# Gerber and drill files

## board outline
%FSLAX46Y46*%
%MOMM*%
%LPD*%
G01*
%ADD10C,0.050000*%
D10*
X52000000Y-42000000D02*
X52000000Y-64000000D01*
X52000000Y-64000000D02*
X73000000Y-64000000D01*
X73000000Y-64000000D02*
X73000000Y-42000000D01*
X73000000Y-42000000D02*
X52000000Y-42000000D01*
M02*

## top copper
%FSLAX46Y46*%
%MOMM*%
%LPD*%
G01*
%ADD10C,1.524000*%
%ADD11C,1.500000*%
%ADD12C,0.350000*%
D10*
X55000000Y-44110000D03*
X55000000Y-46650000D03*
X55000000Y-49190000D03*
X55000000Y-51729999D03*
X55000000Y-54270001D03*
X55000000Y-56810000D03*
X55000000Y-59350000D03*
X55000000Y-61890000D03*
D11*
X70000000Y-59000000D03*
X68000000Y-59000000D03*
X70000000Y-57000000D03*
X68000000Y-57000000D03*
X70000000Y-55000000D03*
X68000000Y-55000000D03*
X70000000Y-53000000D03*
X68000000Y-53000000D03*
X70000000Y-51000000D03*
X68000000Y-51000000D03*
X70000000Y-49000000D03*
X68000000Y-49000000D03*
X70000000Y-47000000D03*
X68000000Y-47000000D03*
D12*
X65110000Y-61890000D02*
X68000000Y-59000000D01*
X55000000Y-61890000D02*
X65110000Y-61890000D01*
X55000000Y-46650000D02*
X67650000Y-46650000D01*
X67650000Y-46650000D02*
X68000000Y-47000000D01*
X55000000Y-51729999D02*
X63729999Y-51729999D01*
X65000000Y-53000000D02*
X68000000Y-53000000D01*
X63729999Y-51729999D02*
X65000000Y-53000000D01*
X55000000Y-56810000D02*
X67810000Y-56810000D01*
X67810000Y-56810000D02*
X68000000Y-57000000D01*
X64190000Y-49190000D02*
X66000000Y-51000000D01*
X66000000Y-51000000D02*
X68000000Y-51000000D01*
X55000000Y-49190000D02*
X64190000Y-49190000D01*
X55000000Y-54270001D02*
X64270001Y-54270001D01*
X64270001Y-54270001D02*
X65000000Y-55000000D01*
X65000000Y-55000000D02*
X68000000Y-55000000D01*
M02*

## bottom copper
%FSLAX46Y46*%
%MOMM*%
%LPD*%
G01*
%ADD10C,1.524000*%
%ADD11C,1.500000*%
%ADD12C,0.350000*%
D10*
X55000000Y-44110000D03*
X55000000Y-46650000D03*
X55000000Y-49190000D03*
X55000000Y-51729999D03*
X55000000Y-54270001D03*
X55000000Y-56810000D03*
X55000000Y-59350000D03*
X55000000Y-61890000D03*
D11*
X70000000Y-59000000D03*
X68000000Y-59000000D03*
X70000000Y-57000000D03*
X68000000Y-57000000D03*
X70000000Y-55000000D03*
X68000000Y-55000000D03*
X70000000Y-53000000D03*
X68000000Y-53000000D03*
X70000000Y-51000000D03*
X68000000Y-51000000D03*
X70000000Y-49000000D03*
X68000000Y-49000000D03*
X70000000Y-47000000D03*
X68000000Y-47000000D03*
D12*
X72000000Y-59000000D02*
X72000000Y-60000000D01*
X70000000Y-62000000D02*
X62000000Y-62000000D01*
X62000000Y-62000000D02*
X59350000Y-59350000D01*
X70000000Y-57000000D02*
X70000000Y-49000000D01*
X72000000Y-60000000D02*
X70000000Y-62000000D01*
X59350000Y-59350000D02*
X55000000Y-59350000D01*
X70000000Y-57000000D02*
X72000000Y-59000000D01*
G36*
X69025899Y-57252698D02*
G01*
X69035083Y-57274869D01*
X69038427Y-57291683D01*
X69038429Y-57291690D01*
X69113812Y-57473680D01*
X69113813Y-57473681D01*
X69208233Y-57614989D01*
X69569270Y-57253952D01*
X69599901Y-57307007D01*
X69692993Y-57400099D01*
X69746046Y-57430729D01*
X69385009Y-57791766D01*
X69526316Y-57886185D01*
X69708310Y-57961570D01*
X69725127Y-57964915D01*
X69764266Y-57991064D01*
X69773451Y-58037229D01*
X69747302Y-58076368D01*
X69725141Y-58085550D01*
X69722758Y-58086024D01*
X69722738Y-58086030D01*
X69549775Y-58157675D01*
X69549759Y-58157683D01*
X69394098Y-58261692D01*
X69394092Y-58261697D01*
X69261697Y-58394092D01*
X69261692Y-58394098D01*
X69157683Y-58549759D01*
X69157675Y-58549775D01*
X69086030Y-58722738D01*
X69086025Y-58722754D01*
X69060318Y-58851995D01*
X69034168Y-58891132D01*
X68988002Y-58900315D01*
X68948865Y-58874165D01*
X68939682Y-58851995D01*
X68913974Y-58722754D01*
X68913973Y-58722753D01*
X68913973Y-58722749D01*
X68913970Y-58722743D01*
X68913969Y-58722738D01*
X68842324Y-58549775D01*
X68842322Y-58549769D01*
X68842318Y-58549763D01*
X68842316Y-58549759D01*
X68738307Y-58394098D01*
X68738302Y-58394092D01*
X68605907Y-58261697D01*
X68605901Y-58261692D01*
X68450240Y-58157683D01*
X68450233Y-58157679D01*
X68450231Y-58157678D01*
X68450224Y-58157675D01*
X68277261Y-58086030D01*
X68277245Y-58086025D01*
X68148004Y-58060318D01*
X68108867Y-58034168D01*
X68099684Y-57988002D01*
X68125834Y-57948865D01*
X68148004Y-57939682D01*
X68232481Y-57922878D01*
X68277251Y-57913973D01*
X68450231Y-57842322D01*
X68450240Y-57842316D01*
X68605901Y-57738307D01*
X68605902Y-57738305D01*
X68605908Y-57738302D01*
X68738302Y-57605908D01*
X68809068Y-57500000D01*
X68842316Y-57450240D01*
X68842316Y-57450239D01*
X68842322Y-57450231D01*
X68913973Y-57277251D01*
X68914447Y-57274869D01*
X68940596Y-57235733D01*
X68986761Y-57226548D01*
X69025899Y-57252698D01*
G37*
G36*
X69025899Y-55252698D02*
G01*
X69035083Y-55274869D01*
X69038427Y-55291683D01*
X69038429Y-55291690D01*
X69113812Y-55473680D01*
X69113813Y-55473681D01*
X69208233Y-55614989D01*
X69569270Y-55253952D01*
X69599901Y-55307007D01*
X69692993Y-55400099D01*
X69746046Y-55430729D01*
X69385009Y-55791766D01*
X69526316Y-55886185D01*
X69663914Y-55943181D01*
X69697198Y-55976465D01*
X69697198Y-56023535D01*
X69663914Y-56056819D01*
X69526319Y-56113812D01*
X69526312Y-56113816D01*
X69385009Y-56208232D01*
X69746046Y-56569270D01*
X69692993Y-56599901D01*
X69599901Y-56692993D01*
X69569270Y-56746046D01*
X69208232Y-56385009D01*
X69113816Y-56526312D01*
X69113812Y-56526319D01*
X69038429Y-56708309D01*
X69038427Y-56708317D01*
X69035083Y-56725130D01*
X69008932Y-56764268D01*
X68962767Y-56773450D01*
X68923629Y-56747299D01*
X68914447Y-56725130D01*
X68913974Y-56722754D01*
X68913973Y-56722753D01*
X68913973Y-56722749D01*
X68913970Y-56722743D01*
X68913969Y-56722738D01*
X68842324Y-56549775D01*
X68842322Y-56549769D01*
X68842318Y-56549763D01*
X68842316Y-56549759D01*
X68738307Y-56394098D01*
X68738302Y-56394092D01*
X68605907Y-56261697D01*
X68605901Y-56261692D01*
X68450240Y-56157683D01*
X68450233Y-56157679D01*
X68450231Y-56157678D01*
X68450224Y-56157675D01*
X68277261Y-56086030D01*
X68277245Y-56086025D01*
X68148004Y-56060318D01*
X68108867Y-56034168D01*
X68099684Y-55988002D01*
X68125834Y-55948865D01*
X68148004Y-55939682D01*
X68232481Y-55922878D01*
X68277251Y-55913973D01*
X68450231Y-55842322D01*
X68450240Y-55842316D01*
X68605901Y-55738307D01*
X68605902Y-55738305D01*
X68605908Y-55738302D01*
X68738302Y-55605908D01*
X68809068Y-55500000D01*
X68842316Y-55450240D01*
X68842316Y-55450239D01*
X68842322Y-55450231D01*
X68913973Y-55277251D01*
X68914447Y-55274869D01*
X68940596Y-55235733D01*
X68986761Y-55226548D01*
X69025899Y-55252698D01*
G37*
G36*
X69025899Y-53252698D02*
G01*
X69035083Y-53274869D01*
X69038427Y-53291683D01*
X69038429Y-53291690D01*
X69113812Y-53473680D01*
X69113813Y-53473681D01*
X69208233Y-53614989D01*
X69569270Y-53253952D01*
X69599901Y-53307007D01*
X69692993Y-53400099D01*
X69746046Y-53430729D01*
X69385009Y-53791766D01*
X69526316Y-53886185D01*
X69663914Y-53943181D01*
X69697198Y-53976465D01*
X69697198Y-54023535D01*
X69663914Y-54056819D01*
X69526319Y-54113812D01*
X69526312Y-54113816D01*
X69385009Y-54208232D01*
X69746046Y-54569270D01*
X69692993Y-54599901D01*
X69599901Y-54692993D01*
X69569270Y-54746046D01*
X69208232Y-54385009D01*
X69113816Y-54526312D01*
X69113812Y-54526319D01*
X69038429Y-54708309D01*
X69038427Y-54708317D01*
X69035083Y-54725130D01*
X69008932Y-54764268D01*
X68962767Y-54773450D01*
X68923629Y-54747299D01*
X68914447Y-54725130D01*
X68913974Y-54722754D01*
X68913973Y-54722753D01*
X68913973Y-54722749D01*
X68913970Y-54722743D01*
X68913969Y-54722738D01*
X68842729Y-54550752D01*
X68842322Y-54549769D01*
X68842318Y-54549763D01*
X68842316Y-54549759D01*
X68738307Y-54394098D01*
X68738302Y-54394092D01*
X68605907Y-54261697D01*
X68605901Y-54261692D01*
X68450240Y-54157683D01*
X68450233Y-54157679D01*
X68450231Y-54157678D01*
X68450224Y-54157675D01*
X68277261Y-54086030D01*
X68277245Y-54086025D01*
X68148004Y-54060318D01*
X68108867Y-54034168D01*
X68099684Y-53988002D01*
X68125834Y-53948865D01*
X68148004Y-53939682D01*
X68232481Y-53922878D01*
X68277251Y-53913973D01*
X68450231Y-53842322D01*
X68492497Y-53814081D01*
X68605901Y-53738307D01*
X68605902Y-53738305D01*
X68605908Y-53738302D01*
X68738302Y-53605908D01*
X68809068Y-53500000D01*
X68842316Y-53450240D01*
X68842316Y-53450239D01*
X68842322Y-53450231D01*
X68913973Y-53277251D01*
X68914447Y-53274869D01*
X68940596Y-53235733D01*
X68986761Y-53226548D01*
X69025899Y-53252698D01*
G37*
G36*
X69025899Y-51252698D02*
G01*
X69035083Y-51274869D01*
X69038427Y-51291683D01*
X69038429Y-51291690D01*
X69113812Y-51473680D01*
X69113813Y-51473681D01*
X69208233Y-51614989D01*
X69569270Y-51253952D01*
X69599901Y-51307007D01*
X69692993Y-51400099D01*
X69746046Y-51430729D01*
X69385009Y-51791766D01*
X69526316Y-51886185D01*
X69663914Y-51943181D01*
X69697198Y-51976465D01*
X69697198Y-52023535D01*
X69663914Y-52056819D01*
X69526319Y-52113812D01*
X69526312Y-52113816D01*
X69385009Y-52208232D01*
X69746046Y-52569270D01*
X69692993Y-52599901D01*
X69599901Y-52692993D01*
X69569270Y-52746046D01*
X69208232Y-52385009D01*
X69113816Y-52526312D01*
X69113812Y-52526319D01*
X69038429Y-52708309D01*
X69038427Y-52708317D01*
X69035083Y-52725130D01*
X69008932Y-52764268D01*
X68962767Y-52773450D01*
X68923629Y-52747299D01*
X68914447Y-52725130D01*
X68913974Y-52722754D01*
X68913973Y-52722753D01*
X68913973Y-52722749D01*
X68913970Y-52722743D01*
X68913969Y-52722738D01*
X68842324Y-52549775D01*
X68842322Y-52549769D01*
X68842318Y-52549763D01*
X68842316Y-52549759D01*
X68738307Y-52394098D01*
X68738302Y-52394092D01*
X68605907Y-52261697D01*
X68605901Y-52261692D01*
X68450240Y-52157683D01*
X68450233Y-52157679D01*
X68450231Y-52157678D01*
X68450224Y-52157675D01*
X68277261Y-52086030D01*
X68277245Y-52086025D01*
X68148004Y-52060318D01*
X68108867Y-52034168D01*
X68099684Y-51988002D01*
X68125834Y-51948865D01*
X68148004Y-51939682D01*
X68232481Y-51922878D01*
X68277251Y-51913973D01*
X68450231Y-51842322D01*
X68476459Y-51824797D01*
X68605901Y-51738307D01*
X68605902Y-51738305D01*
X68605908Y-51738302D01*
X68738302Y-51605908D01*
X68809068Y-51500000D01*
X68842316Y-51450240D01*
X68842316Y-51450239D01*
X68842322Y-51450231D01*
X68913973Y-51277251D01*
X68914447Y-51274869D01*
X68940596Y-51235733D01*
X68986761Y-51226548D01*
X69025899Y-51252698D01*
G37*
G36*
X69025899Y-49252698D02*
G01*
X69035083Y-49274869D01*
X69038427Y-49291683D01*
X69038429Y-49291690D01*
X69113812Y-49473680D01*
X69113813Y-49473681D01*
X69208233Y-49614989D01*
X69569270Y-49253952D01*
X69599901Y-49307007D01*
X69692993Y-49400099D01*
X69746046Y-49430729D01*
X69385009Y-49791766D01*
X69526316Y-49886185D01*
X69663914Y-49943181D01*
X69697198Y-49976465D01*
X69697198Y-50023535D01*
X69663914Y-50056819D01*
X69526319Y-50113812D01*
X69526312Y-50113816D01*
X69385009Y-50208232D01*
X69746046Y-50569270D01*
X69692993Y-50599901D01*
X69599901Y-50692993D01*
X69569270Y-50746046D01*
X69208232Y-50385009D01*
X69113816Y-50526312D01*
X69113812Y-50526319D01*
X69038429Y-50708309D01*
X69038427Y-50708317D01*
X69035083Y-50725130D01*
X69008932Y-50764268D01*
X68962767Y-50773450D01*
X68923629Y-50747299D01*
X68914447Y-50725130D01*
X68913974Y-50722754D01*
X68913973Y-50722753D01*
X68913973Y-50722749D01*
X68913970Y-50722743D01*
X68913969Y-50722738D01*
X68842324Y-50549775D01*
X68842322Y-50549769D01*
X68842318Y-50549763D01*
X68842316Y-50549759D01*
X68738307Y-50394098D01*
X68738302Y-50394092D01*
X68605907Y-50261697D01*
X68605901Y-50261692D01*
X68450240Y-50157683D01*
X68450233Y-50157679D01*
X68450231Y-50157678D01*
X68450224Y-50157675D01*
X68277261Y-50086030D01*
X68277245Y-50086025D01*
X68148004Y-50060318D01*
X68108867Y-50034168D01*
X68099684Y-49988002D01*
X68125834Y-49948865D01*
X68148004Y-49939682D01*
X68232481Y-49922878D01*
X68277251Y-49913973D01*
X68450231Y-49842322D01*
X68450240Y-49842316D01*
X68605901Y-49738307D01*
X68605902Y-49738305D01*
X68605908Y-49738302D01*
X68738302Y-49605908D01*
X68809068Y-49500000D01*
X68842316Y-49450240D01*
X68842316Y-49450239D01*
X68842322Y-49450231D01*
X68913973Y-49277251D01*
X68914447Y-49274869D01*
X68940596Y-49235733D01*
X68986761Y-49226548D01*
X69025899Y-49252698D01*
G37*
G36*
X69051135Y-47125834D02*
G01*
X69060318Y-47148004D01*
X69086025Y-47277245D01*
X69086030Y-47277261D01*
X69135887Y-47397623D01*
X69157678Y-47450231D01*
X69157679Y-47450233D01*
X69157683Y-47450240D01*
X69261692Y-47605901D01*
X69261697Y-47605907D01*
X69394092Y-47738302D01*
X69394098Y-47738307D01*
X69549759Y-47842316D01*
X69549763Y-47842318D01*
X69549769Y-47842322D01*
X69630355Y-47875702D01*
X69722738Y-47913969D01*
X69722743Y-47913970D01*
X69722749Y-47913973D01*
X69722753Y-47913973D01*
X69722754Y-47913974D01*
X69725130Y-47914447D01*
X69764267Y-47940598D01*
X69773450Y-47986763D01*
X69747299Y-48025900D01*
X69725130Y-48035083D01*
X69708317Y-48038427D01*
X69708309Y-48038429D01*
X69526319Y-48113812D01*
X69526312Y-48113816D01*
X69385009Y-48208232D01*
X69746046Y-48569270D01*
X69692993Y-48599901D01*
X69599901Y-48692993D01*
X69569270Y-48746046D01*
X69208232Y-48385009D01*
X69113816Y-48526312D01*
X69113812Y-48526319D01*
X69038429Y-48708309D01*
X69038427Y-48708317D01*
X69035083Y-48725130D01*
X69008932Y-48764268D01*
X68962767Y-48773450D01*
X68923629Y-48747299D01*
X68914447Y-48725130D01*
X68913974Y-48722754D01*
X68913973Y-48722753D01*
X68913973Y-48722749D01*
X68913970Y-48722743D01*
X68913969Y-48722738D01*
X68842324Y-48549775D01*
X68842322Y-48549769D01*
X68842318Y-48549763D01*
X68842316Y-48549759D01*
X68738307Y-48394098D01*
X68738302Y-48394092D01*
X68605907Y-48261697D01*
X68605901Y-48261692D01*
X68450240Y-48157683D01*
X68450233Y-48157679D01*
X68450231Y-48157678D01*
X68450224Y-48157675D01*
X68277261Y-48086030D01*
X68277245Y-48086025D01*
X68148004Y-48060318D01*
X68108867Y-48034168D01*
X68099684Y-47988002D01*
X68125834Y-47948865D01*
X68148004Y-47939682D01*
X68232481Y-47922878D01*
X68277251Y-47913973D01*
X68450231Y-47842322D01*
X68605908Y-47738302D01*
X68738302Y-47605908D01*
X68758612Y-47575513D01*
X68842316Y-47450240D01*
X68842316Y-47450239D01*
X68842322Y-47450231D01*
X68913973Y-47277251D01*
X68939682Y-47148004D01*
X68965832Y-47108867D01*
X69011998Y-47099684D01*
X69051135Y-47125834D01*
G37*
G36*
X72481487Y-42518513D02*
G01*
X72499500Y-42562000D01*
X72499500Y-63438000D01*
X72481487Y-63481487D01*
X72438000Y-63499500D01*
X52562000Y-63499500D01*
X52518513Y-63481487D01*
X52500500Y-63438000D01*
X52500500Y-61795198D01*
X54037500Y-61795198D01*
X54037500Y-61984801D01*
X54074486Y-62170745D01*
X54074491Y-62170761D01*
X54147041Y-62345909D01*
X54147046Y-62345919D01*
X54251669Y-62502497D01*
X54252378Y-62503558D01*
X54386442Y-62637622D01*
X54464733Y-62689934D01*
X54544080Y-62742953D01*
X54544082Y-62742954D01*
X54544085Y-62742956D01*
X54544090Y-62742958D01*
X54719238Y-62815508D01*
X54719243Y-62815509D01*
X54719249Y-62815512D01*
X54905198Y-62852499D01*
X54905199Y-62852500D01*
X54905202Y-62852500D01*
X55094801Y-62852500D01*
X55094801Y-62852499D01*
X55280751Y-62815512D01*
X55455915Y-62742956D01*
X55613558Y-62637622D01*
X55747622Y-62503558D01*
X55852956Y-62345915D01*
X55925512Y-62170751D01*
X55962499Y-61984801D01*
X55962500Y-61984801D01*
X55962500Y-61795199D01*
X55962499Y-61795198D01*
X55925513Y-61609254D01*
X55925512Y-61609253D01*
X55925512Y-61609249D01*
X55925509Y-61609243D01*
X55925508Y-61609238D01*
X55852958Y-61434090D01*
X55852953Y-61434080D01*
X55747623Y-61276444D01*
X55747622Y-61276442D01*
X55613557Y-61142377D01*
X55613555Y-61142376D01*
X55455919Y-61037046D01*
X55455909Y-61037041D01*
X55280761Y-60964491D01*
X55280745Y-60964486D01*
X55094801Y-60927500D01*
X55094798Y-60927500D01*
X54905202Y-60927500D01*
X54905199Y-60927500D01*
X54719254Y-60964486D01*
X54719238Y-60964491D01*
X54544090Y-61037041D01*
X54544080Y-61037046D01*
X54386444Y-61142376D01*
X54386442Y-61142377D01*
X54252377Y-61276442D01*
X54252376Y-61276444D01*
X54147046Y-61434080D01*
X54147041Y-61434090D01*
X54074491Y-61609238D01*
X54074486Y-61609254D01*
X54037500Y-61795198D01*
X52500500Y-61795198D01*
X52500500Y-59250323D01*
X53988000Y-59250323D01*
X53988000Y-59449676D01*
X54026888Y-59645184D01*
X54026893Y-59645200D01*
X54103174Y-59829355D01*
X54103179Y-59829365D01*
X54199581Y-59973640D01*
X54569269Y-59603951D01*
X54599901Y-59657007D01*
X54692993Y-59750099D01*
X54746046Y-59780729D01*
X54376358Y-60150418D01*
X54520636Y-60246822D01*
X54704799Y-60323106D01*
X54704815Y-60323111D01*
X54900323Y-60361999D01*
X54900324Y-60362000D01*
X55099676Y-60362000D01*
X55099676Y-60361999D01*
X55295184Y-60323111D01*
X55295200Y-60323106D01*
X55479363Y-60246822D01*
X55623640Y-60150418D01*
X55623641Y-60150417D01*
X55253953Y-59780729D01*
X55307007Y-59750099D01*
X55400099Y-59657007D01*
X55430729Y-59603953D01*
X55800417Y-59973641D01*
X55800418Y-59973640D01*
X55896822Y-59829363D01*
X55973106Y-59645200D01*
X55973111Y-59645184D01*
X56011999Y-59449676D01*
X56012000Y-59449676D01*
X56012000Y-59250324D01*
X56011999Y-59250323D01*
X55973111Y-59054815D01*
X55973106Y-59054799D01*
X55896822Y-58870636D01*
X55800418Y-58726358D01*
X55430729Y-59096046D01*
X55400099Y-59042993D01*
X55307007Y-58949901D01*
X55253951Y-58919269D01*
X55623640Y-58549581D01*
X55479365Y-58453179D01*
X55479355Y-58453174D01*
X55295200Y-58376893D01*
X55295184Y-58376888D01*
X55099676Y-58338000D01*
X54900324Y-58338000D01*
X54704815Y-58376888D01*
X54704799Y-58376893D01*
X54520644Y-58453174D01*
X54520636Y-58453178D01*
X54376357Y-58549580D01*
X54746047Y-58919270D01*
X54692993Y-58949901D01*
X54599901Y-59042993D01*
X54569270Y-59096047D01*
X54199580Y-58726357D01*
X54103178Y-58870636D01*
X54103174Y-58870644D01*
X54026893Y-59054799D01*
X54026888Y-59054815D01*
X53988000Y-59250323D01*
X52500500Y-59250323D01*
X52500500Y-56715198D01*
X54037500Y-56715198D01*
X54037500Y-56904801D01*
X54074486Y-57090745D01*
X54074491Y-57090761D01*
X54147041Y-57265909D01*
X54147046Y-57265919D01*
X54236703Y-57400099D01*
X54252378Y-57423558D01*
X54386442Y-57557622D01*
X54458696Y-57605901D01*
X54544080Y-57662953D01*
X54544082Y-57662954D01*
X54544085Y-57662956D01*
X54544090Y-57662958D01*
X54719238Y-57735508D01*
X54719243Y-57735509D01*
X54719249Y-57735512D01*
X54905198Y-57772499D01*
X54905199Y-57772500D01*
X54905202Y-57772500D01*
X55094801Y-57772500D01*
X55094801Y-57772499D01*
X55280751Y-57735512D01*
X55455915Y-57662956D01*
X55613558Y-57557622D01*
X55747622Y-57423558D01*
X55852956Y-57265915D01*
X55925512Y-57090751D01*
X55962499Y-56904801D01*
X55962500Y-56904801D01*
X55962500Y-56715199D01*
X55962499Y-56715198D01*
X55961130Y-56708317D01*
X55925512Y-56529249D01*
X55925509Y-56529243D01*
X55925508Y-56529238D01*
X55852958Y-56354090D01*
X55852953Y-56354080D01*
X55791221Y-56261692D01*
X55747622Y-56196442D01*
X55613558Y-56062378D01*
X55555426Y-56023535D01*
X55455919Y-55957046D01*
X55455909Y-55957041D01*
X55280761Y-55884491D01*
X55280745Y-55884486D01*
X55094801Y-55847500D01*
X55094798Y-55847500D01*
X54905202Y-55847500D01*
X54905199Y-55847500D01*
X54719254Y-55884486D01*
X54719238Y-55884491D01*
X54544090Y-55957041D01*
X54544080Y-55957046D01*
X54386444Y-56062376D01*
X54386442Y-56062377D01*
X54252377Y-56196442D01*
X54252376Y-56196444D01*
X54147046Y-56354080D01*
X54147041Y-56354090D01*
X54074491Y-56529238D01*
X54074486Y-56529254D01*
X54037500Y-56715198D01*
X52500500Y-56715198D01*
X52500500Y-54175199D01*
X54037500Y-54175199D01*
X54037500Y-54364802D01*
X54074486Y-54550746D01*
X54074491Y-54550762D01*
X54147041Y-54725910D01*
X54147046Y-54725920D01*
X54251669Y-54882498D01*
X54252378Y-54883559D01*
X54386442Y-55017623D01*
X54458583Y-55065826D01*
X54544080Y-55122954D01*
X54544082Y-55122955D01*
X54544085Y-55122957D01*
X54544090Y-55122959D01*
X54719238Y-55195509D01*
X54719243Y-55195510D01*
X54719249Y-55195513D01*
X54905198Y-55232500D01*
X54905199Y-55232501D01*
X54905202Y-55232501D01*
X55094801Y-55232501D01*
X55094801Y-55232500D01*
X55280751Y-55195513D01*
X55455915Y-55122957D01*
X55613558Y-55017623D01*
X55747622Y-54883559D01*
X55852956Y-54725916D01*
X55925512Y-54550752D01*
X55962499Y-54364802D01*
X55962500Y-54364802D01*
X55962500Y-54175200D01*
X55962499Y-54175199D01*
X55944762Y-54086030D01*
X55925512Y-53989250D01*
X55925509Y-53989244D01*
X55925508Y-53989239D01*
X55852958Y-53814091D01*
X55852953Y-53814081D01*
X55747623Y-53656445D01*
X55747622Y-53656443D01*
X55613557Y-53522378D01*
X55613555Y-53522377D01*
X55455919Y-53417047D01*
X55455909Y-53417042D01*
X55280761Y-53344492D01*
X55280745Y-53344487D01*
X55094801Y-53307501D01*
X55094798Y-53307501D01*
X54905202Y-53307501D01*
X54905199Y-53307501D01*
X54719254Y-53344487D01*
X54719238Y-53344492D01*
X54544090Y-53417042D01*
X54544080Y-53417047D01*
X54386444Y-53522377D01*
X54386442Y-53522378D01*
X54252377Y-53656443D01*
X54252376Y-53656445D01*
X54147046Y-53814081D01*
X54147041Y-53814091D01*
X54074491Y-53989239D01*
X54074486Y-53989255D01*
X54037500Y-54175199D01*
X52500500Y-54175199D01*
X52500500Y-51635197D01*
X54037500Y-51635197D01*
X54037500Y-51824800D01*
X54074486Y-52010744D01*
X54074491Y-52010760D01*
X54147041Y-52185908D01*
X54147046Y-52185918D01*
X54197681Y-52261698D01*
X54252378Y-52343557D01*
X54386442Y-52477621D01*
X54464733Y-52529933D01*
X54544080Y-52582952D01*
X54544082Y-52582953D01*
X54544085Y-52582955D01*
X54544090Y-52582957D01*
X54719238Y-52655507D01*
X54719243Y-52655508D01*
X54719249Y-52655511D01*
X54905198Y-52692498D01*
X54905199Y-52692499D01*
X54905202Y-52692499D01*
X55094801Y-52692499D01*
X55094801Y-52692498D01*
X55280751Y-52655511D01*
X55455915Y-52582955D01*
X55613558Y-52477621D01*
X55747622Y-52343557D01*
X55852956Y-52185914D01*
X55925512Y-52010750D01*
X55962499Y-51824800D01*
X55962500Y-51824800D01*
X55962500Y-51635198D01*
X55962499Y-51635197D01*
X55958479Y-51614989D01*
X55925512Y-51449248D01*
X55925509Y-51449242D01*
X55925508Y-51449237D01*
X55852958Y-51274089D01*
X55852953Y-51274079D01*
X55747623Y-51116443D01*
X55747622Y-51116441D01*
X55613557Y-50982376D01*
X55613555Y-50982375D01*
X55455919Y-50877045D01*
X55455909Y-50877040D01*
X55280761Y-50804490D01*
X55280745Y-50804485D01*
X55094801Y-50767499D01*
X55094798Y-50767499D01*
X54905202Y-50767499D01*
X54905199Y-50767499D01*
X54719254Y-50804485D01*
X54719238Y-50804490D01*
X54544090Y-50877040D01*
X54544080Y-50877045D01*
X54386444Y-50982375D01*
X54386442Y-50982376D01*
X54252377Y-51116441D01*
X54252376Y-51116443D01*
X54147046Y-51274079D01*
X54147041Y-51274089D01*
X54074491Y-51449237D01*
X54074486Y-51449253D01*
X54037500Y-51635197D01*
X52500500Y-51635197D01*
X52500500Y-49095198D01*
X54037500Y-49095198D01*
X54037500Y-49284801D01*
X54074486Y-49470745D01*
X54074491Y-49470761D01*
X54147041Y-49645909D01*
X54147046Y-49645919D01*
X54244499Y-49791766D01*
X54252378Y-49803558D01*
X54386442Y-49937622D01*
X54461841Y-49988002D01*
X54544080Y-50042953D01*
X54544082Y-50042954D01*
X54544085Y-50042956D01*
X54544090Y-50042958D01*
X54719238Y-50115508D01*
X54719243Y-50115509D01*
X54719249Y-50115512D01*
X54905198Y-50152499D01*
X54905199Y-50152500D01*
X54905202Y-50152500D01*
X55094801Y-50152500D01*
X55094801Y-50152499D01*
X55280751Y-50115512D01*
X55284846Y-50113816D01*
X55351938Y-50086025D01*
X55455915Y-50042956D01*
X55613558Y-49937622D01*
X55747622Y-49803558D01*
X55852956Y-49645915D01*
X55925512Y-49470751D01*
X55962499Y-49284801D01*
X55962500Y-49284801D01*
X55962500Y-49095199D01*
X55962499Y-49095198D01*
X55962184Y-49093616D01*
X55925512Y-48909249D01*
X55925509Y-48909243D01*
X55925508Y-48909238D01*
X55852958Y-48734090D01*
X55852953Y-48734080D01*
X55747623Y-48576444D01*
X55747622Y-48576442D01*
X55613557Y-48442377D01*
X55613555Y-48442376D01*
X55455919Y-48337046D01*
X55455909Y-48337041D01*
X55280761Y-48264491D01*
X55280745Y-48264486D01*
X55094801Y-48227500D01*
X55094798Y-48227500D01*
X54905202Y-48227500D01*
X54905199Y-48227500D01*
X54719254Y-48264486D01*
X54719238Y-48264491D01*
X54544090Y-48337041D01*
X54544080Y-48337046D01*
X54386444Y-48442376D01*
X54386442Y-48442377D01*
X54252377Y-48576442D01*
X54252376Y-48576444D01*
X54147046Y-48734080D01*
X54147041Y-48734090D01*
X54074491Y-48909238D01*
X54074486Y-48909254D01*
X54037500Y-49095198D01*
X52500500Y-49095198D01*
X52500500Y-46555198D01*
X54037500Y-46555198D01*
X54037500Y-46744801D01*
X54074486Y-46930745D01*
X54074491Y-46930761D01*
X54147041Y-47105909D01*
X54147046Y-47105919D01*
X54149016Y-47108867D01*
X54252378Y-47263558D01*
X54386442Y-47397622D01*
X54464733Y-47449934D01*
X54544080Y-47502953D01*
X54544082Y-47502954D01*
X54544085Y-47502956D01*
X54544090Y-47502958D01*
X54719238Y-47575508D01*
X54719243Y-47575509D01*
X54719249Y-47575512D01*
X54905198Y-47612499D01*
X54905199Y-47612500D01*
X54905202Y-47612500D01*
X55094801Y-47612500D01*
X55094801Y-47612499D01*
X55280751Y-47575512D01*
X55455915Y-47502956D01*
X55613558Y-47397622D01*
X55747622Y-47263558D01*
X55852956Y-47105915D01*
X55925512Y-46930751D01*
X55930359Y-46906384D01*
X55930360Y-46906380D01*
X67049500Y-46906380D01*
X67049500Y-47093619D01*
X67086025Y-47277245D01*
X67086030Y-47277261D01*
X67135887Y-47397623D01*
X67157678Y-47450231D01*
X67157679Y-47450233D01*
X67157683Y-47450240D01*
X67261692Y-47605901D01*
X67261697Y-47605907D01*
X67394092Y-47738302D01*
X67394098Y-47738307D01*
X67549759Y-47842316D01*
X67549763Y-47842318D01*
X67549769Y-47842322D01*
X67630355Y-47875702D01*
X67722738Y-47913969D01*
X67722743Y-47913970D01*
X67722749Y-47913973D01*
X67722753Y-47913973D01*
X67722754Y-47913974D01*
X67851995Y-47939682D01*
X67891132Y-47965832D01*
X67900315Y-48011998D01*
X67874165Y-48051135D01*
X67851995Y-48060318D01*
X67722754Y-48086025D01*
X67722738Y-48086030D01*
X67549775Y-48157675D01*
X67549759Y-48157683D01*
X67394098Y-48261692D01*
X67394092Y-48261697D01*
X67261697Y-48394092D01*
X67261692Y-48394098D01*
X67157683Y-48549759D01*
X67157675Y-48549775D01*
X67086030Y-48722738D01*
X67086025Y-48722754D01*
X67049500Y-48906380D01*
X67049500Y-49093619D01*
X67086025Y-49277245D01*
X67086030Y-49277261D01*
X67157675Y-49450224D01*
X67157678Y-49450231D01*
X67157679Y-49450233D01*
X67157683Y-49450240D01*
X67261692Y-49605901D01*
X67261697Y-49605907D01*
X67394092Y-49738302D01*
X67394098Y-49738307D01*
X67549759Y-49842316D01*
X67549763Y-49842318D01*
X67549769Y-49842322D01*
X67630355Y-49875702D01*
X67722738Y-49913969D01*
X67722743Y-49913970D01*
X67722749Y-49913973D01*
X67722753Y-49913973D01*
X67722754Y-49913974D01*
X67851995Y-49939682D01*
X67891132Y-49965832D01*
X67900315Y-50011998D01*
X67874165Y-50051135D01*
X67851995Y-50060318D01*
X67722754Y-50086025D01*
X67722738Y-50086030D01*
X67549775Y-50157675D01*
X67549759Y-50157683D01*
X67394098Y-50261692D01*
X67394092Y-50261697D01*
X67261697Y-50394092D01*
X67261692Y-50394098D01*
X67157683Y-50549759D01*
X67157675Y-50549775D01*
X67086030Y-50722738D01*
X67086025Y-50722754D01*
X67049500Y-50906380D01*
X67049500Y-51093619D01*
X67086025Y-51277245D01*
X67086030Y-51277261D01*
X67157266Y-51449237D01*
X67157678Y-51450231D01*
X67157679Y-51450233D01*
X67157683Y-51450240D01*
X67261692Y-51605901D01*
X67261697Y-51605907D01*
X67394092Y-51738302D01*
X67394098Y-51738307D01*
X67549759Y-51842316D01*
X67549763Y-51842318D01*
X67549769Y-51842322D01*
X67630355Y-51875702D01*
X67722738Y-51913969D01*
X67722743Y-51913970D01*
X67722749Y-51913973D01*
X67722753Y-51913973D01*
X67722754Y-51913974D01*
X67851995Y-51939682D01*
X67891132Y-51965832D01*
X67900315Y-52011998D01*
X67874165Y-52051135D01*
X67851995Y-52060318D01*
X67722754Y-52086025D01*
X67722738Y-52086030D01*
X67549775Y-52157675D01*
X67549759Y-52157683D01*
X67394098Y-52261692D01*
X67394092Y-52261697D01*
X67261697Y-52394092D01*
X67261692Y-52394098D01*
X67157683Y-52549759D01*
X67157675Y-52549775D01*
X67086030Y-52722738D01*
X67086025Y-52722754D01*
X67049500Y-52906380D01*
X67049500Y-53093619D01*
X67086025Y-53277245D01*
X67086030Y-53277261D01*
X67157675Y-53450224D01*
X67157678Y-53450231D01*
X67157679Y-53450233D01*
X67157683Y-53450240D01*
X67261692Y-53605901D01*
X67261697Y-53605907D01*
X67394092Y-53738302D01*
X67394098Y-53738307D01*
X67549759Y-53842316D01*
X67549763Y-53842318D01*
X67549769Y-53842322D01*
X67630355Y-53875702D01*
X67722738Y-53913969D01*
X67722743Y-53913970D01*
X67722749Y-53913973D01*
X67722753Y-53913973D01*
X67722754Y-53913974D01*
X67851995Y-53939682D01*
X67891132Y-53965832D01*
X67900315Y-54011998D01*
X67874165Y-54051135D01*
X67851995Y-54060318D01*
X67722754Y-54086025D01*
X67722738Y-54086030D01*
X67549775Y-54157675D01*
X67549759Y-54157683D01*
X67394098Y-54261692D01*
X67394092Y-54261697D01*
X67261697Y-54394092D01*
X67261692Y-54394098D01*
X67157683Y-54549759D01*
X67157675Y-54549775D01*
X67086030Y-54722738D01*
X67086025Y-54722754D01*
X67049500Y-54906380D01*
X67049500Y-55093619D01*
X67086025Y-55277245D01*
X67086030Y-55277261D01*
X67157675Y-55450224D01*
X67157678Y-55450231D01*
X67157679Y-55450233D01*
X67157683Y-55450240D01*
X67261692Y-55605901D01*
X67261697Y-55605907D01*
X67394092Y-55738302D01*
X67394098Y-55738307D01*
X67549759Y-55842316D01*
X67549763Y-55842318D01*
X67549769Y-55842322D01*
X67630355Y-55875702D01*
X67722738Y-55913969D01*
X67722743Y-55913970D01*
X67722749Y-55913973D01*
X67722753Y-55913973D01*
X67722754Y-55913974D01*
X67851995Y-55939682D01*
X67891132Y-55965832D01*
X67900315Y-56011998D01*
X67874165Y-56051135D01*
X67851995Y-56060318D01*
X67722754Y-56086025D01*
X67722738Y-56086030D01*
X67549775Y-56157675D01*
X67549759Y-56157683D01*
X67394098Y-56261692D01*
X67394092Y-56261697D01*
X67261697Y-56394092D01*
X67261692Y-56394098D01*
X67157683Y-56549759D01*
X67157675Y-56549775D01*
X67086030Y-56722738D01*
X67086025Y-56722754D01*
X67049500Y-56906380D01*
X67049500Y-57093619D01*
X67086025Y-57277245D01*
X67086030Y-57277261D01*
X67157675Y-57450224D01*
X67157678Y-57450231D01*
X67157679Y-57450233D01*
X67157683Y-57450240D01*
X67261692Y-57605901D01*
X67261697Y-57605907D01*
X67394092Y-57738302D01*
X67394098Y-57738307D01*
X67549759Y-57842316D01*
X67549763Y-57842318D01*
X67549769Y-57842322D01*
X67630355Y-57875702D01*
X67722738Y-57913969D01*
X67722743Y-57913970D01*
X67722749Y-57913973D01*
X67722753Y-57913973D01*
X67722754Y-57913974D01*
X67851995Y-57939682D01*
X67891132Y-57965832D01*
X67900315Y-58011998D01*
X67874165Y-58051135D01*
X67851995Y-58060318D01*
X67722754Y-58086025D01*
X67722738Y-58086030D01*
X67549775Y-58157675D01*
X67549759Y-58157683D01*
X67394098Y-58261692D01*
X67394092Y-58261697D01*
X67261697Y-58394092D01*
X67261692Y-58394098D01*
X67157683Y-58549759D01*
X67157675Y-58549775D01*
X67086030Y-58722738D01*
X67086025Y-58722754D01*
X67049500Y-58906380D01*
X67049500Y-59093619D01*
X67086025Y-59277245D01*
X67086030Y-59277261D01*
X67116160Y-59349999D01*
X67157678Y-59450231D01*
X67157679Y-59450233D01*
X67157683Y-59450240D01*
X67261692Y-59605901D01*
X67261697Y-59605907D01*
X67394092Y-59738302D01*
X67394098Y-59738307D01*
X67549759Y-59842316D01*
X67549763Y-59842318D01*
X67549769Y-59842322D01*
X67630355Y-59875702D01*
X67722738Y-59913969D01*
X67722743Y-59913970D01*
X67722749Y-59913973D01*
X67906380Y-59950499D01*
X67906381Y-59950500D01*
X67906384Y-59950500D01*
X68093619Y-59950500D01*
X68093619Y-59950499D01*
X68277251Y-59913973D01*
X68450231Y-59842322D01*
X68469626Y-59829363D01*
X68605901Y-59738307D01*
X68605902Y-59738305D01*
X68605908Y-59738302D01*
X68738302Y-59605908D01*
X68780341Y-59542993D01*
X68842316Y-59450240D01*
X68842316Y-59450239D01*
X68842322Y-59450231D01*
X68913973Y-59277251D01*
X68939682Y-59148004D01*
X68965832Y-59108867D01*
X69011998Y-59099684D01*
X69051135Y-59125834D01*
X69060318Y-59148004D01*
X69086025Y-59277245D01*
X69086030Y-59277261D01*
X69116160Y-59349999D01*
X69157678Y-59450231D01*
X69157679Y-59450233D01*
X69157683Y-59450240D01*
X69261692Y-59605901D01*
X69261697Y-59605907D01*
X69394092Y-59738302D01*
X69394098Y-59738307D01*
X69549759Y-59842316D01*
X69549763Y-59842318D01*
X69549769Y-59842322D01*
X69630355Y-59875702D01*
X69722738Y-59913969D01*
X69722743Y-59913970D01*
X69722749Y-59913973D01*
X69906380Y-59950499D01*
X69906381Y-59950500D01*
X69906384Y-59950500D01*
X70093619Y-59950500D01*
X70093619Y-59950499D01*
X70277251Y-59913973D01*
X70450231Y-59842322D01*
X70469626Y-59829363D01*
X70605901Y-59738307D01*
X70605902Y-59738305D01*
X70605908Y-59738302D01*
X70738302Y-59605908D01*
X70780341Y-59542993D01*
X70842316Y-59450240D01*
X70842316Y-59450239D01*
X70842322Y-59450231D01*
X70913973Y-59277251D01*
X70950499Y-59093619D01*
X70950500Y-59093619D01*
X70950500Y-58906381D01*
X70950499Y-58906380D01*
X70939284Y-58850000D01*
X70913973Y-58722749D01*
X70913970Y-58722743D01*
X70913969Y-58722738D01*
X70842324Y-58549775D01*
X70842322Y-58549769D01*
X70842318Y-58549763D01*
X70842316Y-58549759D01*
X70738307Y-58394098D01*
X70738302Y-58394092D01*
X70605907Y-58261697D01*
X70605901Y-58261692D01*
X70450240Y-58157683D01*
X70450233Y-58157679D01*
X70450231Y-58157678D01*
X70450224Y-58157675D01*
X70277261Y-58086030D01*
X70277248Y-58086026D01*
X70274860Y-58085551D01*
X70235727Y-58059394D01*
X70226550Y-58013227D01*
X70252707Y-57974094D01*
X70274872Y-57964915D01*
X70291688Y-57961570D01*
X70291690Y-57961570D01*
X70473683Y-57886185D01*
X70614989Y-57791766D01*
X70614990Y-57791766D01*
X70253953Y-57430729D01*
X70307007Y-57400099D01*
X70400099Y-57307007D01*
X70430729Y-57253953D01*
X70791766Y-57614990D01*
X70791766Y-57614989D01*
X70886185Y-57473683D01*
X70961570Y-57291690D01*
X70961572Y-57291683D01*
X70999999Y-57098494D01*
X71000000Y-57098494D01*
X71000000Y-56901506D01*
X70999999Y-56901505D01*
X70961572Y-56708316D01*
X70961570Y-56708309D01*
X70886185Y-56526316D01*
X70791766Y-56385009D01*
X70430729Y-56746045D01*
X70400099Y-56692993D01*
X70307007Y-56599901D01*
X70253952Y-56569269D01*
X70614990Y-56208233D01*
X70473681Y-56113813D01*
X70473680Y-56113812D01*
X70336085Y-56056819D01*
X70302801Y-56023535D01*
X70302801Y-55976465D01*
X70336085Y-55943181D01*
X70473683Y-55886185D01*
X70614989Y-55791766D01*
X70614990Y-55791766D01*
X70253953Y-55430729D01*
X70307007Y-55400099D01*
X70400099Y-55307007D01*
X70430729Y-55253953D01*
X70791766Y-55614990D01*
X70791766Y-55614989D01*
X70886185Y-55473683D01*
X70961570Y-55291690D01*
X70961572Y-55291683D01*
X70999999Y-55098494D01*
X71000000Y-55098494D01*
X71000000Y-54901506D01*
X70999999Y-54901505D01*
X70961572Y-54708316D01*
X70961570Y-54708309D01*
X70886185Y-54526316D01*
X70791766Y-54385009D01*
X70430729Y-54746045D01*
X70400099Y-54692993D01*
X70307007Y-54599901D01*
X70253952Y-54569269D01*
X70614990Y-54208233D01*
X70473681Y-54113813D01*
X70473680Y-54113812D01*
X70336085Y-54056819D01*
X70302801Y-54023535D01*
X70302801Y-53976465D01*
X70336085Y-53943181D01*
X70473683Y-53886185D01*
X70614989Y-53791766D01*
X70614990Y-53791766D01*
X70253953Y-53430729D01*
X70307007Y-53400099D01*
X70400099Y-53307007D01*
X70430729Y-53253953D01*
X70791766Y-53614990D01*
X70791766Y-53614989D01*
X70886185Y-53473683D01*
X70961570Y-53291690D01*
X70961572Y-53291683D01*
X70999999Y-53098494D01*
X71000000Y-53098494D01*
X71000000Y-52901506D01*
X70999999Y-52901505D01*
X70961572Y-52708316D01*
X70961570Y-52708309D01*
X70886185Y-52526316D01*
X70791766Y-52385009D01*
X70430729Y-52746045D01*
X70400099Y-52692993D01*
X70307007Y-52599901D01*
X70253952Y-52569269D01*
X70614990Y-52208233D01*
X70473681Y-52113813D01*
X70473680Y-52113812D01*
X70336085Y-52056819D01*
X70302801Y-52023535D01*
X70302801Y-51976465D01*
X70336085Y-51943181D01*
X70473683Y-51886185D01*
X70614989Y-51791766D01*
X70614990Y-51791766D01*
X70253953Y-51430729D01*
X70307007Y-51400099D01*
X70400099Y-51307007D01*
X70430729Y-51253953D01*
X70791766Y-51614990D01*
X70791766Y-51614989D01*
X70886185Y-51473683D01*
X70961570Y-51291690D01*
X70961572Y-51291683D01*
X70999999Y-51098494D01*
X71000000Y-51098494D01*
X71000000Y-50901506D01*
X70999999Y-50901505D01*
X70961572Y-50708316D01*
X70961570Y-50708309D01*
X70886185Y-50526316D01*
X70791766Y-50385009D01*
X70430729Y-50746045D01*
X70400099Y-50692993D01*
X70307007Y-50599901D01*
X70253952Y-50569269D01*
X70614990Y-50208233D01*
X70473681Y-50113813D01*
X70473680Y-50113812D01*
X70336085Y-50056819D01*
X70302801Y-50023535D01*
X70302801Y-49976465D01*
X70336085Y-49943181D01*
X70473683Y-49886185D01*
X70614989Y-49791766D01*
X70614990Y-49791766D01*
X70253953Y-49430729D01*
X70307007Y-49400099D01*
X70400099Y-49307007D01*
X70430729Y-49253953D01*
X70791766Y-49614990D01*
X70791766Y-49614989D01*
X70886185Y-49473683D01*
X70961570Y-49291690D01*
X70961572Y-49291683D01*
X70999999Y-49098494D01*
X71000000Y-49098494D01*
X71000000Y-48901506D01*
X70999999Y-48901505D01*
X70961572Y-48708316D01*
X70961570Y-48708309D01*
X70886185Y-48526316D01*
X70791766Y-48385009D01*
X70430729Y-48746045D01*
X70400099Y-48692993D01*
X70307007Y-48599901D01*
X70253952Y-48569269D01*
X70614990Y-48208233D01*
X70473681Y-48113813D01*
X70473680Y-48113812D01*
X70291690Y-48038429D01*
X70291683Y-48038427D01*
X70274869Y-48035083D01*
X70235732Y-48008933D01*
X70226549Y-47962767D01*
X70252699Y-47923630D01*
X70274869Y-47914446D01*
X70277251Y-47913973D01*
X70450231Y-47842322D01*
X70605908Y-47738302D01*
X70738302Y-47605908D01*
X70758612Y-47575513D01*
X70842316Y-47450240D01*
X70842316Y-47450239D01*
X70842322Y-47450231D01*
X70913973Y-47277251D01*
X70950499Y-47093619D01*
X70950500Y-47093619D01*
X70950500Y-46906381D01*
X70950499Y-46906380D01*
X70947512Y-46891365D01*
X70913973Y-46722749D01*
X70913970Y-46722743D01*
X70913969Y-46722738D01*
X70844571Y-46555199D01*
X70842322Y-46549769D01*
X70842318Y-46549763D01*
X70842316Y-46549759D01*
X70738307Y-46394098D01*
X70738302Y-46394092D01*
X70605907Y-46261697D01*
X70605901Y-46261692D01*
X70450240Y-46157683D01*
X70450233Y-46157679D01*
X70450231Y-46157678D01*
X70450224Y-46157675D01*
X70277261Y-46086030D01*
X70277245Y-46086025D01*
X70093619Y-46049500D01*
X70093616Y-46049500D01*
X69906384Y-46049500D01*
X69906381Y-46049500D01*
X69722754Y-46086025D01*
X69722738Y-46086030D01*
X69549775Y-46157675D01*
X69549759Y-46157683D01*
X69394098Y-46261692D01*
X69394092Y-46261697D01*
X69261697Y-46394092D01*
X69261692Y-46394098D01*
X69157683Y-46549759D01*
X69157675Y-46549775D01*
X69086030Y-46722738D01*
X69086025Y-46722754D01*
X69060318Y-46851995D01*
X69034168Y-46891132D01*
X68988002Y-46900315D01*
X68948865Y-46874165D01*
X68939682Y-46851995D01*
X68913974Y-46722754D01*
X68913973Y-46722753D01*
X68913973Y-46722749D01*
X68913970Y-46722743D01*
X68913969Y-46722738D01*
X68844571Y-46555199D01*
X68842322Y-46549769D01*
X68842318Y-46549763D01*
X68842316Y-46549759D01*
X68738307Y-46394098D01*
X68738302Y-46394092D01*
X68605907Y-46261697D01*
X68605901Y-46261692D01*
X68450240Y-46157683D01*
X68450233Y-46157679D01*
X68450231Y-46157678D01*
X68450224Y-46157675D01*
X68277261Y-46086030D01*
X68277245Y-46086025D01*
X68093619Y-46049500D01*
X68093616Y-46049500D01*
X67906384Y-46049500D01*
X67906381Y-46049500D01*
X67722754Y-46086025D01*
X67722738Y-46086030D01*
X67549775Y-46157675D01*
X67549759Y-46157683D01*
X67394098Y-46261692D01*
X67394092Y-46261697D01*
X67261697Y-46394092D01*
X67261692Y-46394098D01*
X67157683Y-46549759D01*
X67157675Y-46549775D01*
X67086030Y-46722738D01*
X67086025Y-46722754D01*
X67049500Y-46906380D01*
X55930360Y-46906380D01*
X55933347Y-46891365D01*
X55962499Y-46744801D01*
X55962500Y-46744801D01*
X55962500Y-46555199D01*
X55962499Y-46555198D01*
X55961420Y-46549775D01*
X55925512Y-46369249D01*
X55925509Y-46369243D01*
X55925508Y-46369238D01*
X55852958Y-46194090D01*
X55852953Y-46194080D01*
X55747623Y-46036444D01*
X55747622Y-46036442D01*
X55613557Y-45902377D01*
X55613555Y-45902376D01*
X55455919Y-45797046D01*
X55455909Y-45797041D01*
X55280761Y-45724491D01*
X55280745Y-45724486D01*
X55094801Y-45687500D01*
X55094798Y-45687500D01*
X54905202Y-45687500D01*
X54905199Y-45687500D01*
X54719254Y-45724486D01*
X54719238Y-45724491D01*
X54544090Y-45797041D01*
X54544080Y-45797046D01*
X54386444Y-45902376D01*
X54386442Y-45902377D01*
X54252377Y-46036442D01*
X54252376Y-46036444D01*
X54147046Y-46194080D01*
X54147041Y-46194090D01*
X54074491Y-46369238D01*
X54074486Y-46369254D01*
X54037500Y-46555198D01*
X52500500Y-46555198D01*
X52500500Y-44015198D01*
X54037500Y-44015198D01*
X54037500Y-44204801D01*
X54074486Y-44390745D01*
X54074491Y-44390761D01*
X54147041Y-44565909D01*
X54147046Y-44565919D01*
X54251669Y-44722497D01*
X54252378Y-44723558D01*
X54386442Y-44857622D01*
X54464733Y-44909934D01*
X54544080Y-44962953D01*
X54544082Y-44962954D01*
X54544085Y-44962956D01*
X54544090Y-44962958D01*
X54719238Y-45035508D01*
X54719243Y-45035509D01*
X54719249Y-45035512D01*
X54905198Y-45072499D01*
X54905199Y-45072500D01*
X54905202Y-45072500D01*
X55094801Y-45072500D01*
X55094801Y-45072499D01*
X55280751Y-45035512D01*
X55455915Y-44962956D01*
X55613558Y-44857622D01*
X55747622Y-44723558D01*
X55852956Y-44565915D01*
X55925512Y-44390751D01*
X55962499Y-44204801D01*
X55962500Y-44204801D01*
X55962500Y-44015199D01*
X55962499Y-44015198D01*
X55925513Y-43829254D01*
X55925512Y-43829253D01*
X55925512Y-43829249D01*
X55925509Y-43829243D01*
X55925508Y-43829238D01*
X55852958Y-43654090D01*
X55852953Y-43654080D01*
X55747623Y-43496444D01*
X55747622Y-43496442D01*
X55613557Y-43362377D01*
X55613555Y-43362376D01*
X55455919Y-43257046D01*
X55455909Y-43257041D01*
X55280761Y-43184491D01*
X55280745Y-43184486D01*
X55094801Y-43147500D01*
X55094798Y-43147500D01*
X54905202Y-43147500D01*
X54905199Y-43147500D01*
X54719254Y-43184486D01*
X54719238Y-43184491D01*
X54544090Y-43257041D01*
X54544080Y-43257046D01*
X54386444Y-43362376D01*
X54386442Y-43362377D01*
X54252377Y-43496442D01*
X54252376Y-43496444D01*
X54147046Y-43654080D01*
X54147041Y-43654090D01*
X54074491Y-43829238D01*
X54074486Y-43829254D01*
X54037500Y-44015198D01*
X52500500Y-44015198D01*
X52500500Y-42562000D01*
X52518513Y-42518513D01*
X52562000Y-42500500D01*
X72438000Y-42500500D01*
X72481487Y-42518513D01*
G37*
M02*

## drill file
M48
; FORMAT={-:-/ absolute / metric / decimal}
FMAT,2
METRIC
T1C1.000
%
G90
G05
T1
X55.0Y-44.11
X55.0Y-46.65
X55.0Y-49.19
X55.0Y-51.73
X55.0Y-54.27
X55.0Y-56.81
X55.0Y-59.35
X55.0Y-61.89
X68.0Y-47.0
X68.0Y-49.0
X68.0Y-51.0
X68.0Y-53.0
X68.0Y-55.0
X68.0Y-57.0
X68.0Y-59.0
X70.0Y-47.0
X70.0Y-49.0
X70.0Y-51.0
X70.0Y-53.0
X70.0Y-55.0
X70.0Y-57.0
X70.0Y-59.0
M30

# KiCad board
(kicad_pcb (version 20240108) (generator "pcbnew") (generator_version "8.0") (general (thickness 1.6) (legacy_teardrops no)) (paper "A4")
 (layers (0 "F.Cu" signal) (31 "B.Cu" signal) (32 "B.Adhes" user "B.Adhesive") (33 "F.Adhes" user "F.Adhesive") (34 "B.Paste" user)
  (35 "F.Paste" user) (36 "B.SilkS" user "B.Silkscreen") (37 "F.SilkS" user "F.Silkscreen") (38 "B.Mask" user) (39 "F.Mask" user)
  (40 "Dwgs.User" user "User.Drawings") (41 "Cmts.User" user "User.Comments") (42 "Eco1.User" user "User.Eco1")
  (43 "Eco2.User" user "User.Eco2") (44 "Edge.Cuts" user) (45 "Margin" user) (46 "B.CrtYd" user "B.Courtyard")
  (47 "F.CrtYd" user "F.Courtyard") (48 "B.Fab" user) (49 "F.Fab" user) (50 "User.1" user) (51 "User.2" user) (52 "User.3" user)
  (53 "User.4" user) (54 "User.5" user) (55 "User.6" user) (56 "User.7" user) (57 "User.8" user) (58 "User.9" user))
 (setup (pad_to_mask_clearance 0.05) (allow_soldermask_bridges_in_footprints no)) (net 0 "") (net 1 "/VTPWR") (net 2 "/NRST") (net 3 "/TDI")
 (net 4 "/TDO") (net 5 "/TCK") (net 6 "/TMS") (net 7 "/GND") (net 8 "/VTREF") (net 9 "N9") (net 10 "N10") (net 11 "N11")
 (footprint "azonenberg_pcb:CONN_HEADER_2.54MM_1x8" (layer "F.Cu") (at 55 53 -90)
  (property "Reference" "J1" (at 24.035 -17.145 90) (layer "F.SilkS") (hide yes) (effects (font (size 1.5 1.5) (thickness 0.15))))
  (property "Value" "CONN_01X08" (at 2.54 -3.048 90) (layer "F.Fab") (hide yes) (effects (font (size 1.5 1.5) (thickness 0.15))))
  (pad "1" thru_hole circle (at -8.89 0 270) (size 1.524 1.524) (drill 1) (layers "*.Cu" "*.Mask") (remove_unused_layers no)
   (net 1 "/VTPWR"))
  (pad "2" thru_hole circle (at -6.35 0) (size 1.524 1.524) (drill 1) (layers "*.Cu" "*.Mask") (remove_unused_layers no) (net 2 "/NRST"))
  (pad "3" thru_hole circle (at -3.81 0 270) (size 1.524 1.524) (drill 1) (layers "*.Cu" "*.Mask") (remove_unused_layers no) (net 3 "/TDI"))
  (pad "4" thru_hole circle (at -1.270001 0 270) (size 1.524 1.524) (drill 1) (layers "*.Cu" "*.Mask") (remove_unused_layers no)
   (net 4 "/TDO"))
  (pad "5" thru_hole circle (at 1.270001 0 270) (size 1.524 1.524) (drill 1) (layers "*.Cu" "*.Mask") (remove_unused_layers no)
   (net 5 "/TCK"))
  (pad "6" thru_hole circle (at 3.81 0 270) (size 1.524 1.524) (drill 1) (layers "*.Cu" "*.Mask") (remove_unused_layers no) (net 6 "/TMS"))
  (pad "7" thru_hole circle (at 6.35 0 270) (size 1.524 1.524) (drill 1) (layers "*.Cu" "*.Mask") (remove_unused_layers no) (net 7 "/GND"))
  (pad "8" thru_hole circle (at 8.89 0 270) (size 1.524 1.524) (drill 1) (layers "*.Cu" "*.Mask") (remove_unused_layers no) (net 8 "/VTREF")))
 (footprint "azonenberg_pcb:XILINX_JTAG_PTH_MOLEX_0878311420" (layer "F.Cu") (at 69 53 90)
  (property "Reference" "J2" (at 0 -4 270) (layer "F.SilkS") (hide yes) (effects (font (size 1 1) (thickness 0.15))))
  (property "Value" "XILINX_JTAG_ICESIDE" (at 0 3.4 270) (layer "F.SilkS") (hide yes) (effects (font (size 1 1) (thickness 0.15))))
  (pad "1" thru_hole circle (at -6 1 90) (size 1.5 1.5) (drill 1) (layers "*.Cu" "*.Mask" "F.Paste") (remove_unused_layers no) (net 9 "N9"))
  (pad "2" thru_hole circle (at -6 -1 90) (size 1.5 1.5) (drill 1) (layers "*.Cu" "*.Mask" "F.Paste") (remove_unused_layers no)
   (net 8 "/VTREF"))
  (pad "3" thru_hole circle (at -4 1 90) (size 1.5 1.5) (drill 1) (layers "*.Cu" "*.Mask" "F.Paste") (remove_unused_layers no)
   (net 7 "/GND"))
  (pad "4" thru_hole circle (at -4 -1 90) (size 1.5 1.5) (drill 1) (layers "*.Cu" "*.Mask" "F.Paste") (remove_unused_layers no)
   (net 6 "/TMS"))
  (pad "5" thru_hole circle (at -2 1 90) (size 1.5 1.5) (drill 1) (layers "*.Cu" "*.Mask" "F.Paste") (remove_unused_layers no)
   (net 7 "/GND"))
  (pad "6" thru_hole circle (at -2 -1 90) (size 1.5 1.5) (drill 1) (layers "*.Cu" "*.Mask" "F.Paste") (remove_unused_layers no)
   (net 5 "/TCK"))
  (pad "7" thru_hole circle (at 0 1 90) (size 1.5 1.5) (drill 1) (layers "*.Cu" "*.Mask" "F.Paste") (remove_unused_layers no) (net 7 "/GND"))
  (pad "8" thru_hole circle (at 0 -1 90) (size 1.5 1.5) (drill 1) (layers "*.Cu" "*.Mask" "F.Paste") (remove_unused_layers no)
   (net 4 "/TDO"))
  (pad "9" thru_hole circle (at 2 1 90) (size 1.5 1.5) (drill 1) (layers "*.Cu" "*.Mask" "F.Paste") (remove_unused_layers no) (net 7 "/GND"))
  (pad "10" thru_hole circle (at 2 -1 90) (size 1.5 1.5) (drill 1) (layers "*.Cu" "*.Mask" "F.Paste") (remove_unused_layers no)
   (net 3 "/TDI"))
  (pad "11" thru_hole circle (at 4 1 90) (size 1.5 1.5) (drill 1) (layers "*.Cu" "*.Mask" "F.Paste") (remove_unused_layers no)
   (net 7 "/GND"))
  (pad "12" thru_hole circle (at 4 -1 90) (size 1.5 1.5) (drill 1) (layers "*.Cu" "*.Mask" "F.Paste") (remove_unused_layers no)
   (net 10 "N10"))
  (pad "13" thru_hole circle (at 6 1 90) (size 1.5 1.5) (drill 1) (layers "*.Cu" "*.Mask" "F.Paste") (remove_unused_layers no)
   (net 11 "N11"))
  (pad "14" thru_hole circle (at 6 -1 90) (size 1.5 1.5) (drill 1) (layers "*.Cu" "*.Mask" "F.Paste") (remove_unused_layers no)
   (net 2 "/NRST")))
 (gr_line (start 52 42) (end 52 64) (stroke (width 0.05) (type default)) (layer "Edge.Cuts"))
 (gr_line (start 52 64) (end 73 64) (stroke (width 0.05) (type default)) (layer "Edge.Cuts"))
 (gr_line (start 73 64) (end 73 42) (stroke (width 0.05) (type default)) (layer "Edge.Cuts"))
 (gr_line (start 73 42) (end 52 42) (stroke (width 0.05) (type default)) (layer "Edge.Cuts"))
 (segment (start 65.11 61.89) (end 68 59) (width 0.35) (layer "F.Cu") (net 8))
 (segment (start 55 61.89) (end 65.11 61.89) (width 0.35) (layer "F.Cu") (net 8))
 (segment (start 72 59) (end 72 60) (width 0.35) (layer "B.Cu") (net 7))
 (segment (start 70 62) (end 62 62) (width 0.35) (layer "B.Cu") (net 7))
 (segment (start 62 62) (end 59.35 59.35) (width 0.35) (layer "B.Cu") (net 7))
 (segment (start 70 57) (end 70 49) (width 0.35) (layer "B.Cu") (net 7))
 (segment (start 72 60) (end 70 62) (width 0.35) (layer "B.Cu") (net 7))
 (segment (start 59.35 59.35) (end 55 59.35) (width 0.35) (layer "B.Cu") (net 7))
 (segment (start 70 57) (end 72 59) (width 0.35) (layer "B.Cu") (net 7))
 (segment (start 55 46.65) (end 67.65 46.65) (width 0.35) (layer "F.Cu") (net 2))
 (segment (start 67.65 46.65) (end 68 47) (width 0.35) (layer "F.Cu") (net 2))
 (segment (start 55 51.729999) (end 63.729999 51.729999) (width 0.35) (layer "F.Cu") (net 4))
 (segment (start 65 53) (end 68 53) (width 0.35) (layer "F.Cu") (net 4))
 (segment (start 63.729999 51.729999) (end 65 53) (width 0.35) (layer "F.Cu") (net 4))
 (segment (start 55 56.81) (end 67.81 56.81) (width 0.35) (layer "F.Cu") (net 6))
 (segment (start 67.81 56.81) (end 68 57) (width 0.35) (layer "F.Cu") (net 6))
 (segment (start 64.19 49.19) (end 66 51) (width 0.35) (layer "F.Cu") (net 3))
 (segment (start 66 51) (end 68 51) (width 0.35) (layer "F.Cu") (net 3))
 (segment (start 55 49.19) (end 64.19 49.19) (width 0.35) (layer "F.Cu") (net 3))
 (segment (start 55 54.270001) (end 64.270001 54.270001) (width 0.35) (layer "F.Cu") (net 5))
 (segment (start 64.270001 54.270001) (end 65 55) (width 0.35) (layer "F.Cu") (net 5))
 (segment (start 65 55) (end 68 55) (width 0.35) (layer "F.Cu") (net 5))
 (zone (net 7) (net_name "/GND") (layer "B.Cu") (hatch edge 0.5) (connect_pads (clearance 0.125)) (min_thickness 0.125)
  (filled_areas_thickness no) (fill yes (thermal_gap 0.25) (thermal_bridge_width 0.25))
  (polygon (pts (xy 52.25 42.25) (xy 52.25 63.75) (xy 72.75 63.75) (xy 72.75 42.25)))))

